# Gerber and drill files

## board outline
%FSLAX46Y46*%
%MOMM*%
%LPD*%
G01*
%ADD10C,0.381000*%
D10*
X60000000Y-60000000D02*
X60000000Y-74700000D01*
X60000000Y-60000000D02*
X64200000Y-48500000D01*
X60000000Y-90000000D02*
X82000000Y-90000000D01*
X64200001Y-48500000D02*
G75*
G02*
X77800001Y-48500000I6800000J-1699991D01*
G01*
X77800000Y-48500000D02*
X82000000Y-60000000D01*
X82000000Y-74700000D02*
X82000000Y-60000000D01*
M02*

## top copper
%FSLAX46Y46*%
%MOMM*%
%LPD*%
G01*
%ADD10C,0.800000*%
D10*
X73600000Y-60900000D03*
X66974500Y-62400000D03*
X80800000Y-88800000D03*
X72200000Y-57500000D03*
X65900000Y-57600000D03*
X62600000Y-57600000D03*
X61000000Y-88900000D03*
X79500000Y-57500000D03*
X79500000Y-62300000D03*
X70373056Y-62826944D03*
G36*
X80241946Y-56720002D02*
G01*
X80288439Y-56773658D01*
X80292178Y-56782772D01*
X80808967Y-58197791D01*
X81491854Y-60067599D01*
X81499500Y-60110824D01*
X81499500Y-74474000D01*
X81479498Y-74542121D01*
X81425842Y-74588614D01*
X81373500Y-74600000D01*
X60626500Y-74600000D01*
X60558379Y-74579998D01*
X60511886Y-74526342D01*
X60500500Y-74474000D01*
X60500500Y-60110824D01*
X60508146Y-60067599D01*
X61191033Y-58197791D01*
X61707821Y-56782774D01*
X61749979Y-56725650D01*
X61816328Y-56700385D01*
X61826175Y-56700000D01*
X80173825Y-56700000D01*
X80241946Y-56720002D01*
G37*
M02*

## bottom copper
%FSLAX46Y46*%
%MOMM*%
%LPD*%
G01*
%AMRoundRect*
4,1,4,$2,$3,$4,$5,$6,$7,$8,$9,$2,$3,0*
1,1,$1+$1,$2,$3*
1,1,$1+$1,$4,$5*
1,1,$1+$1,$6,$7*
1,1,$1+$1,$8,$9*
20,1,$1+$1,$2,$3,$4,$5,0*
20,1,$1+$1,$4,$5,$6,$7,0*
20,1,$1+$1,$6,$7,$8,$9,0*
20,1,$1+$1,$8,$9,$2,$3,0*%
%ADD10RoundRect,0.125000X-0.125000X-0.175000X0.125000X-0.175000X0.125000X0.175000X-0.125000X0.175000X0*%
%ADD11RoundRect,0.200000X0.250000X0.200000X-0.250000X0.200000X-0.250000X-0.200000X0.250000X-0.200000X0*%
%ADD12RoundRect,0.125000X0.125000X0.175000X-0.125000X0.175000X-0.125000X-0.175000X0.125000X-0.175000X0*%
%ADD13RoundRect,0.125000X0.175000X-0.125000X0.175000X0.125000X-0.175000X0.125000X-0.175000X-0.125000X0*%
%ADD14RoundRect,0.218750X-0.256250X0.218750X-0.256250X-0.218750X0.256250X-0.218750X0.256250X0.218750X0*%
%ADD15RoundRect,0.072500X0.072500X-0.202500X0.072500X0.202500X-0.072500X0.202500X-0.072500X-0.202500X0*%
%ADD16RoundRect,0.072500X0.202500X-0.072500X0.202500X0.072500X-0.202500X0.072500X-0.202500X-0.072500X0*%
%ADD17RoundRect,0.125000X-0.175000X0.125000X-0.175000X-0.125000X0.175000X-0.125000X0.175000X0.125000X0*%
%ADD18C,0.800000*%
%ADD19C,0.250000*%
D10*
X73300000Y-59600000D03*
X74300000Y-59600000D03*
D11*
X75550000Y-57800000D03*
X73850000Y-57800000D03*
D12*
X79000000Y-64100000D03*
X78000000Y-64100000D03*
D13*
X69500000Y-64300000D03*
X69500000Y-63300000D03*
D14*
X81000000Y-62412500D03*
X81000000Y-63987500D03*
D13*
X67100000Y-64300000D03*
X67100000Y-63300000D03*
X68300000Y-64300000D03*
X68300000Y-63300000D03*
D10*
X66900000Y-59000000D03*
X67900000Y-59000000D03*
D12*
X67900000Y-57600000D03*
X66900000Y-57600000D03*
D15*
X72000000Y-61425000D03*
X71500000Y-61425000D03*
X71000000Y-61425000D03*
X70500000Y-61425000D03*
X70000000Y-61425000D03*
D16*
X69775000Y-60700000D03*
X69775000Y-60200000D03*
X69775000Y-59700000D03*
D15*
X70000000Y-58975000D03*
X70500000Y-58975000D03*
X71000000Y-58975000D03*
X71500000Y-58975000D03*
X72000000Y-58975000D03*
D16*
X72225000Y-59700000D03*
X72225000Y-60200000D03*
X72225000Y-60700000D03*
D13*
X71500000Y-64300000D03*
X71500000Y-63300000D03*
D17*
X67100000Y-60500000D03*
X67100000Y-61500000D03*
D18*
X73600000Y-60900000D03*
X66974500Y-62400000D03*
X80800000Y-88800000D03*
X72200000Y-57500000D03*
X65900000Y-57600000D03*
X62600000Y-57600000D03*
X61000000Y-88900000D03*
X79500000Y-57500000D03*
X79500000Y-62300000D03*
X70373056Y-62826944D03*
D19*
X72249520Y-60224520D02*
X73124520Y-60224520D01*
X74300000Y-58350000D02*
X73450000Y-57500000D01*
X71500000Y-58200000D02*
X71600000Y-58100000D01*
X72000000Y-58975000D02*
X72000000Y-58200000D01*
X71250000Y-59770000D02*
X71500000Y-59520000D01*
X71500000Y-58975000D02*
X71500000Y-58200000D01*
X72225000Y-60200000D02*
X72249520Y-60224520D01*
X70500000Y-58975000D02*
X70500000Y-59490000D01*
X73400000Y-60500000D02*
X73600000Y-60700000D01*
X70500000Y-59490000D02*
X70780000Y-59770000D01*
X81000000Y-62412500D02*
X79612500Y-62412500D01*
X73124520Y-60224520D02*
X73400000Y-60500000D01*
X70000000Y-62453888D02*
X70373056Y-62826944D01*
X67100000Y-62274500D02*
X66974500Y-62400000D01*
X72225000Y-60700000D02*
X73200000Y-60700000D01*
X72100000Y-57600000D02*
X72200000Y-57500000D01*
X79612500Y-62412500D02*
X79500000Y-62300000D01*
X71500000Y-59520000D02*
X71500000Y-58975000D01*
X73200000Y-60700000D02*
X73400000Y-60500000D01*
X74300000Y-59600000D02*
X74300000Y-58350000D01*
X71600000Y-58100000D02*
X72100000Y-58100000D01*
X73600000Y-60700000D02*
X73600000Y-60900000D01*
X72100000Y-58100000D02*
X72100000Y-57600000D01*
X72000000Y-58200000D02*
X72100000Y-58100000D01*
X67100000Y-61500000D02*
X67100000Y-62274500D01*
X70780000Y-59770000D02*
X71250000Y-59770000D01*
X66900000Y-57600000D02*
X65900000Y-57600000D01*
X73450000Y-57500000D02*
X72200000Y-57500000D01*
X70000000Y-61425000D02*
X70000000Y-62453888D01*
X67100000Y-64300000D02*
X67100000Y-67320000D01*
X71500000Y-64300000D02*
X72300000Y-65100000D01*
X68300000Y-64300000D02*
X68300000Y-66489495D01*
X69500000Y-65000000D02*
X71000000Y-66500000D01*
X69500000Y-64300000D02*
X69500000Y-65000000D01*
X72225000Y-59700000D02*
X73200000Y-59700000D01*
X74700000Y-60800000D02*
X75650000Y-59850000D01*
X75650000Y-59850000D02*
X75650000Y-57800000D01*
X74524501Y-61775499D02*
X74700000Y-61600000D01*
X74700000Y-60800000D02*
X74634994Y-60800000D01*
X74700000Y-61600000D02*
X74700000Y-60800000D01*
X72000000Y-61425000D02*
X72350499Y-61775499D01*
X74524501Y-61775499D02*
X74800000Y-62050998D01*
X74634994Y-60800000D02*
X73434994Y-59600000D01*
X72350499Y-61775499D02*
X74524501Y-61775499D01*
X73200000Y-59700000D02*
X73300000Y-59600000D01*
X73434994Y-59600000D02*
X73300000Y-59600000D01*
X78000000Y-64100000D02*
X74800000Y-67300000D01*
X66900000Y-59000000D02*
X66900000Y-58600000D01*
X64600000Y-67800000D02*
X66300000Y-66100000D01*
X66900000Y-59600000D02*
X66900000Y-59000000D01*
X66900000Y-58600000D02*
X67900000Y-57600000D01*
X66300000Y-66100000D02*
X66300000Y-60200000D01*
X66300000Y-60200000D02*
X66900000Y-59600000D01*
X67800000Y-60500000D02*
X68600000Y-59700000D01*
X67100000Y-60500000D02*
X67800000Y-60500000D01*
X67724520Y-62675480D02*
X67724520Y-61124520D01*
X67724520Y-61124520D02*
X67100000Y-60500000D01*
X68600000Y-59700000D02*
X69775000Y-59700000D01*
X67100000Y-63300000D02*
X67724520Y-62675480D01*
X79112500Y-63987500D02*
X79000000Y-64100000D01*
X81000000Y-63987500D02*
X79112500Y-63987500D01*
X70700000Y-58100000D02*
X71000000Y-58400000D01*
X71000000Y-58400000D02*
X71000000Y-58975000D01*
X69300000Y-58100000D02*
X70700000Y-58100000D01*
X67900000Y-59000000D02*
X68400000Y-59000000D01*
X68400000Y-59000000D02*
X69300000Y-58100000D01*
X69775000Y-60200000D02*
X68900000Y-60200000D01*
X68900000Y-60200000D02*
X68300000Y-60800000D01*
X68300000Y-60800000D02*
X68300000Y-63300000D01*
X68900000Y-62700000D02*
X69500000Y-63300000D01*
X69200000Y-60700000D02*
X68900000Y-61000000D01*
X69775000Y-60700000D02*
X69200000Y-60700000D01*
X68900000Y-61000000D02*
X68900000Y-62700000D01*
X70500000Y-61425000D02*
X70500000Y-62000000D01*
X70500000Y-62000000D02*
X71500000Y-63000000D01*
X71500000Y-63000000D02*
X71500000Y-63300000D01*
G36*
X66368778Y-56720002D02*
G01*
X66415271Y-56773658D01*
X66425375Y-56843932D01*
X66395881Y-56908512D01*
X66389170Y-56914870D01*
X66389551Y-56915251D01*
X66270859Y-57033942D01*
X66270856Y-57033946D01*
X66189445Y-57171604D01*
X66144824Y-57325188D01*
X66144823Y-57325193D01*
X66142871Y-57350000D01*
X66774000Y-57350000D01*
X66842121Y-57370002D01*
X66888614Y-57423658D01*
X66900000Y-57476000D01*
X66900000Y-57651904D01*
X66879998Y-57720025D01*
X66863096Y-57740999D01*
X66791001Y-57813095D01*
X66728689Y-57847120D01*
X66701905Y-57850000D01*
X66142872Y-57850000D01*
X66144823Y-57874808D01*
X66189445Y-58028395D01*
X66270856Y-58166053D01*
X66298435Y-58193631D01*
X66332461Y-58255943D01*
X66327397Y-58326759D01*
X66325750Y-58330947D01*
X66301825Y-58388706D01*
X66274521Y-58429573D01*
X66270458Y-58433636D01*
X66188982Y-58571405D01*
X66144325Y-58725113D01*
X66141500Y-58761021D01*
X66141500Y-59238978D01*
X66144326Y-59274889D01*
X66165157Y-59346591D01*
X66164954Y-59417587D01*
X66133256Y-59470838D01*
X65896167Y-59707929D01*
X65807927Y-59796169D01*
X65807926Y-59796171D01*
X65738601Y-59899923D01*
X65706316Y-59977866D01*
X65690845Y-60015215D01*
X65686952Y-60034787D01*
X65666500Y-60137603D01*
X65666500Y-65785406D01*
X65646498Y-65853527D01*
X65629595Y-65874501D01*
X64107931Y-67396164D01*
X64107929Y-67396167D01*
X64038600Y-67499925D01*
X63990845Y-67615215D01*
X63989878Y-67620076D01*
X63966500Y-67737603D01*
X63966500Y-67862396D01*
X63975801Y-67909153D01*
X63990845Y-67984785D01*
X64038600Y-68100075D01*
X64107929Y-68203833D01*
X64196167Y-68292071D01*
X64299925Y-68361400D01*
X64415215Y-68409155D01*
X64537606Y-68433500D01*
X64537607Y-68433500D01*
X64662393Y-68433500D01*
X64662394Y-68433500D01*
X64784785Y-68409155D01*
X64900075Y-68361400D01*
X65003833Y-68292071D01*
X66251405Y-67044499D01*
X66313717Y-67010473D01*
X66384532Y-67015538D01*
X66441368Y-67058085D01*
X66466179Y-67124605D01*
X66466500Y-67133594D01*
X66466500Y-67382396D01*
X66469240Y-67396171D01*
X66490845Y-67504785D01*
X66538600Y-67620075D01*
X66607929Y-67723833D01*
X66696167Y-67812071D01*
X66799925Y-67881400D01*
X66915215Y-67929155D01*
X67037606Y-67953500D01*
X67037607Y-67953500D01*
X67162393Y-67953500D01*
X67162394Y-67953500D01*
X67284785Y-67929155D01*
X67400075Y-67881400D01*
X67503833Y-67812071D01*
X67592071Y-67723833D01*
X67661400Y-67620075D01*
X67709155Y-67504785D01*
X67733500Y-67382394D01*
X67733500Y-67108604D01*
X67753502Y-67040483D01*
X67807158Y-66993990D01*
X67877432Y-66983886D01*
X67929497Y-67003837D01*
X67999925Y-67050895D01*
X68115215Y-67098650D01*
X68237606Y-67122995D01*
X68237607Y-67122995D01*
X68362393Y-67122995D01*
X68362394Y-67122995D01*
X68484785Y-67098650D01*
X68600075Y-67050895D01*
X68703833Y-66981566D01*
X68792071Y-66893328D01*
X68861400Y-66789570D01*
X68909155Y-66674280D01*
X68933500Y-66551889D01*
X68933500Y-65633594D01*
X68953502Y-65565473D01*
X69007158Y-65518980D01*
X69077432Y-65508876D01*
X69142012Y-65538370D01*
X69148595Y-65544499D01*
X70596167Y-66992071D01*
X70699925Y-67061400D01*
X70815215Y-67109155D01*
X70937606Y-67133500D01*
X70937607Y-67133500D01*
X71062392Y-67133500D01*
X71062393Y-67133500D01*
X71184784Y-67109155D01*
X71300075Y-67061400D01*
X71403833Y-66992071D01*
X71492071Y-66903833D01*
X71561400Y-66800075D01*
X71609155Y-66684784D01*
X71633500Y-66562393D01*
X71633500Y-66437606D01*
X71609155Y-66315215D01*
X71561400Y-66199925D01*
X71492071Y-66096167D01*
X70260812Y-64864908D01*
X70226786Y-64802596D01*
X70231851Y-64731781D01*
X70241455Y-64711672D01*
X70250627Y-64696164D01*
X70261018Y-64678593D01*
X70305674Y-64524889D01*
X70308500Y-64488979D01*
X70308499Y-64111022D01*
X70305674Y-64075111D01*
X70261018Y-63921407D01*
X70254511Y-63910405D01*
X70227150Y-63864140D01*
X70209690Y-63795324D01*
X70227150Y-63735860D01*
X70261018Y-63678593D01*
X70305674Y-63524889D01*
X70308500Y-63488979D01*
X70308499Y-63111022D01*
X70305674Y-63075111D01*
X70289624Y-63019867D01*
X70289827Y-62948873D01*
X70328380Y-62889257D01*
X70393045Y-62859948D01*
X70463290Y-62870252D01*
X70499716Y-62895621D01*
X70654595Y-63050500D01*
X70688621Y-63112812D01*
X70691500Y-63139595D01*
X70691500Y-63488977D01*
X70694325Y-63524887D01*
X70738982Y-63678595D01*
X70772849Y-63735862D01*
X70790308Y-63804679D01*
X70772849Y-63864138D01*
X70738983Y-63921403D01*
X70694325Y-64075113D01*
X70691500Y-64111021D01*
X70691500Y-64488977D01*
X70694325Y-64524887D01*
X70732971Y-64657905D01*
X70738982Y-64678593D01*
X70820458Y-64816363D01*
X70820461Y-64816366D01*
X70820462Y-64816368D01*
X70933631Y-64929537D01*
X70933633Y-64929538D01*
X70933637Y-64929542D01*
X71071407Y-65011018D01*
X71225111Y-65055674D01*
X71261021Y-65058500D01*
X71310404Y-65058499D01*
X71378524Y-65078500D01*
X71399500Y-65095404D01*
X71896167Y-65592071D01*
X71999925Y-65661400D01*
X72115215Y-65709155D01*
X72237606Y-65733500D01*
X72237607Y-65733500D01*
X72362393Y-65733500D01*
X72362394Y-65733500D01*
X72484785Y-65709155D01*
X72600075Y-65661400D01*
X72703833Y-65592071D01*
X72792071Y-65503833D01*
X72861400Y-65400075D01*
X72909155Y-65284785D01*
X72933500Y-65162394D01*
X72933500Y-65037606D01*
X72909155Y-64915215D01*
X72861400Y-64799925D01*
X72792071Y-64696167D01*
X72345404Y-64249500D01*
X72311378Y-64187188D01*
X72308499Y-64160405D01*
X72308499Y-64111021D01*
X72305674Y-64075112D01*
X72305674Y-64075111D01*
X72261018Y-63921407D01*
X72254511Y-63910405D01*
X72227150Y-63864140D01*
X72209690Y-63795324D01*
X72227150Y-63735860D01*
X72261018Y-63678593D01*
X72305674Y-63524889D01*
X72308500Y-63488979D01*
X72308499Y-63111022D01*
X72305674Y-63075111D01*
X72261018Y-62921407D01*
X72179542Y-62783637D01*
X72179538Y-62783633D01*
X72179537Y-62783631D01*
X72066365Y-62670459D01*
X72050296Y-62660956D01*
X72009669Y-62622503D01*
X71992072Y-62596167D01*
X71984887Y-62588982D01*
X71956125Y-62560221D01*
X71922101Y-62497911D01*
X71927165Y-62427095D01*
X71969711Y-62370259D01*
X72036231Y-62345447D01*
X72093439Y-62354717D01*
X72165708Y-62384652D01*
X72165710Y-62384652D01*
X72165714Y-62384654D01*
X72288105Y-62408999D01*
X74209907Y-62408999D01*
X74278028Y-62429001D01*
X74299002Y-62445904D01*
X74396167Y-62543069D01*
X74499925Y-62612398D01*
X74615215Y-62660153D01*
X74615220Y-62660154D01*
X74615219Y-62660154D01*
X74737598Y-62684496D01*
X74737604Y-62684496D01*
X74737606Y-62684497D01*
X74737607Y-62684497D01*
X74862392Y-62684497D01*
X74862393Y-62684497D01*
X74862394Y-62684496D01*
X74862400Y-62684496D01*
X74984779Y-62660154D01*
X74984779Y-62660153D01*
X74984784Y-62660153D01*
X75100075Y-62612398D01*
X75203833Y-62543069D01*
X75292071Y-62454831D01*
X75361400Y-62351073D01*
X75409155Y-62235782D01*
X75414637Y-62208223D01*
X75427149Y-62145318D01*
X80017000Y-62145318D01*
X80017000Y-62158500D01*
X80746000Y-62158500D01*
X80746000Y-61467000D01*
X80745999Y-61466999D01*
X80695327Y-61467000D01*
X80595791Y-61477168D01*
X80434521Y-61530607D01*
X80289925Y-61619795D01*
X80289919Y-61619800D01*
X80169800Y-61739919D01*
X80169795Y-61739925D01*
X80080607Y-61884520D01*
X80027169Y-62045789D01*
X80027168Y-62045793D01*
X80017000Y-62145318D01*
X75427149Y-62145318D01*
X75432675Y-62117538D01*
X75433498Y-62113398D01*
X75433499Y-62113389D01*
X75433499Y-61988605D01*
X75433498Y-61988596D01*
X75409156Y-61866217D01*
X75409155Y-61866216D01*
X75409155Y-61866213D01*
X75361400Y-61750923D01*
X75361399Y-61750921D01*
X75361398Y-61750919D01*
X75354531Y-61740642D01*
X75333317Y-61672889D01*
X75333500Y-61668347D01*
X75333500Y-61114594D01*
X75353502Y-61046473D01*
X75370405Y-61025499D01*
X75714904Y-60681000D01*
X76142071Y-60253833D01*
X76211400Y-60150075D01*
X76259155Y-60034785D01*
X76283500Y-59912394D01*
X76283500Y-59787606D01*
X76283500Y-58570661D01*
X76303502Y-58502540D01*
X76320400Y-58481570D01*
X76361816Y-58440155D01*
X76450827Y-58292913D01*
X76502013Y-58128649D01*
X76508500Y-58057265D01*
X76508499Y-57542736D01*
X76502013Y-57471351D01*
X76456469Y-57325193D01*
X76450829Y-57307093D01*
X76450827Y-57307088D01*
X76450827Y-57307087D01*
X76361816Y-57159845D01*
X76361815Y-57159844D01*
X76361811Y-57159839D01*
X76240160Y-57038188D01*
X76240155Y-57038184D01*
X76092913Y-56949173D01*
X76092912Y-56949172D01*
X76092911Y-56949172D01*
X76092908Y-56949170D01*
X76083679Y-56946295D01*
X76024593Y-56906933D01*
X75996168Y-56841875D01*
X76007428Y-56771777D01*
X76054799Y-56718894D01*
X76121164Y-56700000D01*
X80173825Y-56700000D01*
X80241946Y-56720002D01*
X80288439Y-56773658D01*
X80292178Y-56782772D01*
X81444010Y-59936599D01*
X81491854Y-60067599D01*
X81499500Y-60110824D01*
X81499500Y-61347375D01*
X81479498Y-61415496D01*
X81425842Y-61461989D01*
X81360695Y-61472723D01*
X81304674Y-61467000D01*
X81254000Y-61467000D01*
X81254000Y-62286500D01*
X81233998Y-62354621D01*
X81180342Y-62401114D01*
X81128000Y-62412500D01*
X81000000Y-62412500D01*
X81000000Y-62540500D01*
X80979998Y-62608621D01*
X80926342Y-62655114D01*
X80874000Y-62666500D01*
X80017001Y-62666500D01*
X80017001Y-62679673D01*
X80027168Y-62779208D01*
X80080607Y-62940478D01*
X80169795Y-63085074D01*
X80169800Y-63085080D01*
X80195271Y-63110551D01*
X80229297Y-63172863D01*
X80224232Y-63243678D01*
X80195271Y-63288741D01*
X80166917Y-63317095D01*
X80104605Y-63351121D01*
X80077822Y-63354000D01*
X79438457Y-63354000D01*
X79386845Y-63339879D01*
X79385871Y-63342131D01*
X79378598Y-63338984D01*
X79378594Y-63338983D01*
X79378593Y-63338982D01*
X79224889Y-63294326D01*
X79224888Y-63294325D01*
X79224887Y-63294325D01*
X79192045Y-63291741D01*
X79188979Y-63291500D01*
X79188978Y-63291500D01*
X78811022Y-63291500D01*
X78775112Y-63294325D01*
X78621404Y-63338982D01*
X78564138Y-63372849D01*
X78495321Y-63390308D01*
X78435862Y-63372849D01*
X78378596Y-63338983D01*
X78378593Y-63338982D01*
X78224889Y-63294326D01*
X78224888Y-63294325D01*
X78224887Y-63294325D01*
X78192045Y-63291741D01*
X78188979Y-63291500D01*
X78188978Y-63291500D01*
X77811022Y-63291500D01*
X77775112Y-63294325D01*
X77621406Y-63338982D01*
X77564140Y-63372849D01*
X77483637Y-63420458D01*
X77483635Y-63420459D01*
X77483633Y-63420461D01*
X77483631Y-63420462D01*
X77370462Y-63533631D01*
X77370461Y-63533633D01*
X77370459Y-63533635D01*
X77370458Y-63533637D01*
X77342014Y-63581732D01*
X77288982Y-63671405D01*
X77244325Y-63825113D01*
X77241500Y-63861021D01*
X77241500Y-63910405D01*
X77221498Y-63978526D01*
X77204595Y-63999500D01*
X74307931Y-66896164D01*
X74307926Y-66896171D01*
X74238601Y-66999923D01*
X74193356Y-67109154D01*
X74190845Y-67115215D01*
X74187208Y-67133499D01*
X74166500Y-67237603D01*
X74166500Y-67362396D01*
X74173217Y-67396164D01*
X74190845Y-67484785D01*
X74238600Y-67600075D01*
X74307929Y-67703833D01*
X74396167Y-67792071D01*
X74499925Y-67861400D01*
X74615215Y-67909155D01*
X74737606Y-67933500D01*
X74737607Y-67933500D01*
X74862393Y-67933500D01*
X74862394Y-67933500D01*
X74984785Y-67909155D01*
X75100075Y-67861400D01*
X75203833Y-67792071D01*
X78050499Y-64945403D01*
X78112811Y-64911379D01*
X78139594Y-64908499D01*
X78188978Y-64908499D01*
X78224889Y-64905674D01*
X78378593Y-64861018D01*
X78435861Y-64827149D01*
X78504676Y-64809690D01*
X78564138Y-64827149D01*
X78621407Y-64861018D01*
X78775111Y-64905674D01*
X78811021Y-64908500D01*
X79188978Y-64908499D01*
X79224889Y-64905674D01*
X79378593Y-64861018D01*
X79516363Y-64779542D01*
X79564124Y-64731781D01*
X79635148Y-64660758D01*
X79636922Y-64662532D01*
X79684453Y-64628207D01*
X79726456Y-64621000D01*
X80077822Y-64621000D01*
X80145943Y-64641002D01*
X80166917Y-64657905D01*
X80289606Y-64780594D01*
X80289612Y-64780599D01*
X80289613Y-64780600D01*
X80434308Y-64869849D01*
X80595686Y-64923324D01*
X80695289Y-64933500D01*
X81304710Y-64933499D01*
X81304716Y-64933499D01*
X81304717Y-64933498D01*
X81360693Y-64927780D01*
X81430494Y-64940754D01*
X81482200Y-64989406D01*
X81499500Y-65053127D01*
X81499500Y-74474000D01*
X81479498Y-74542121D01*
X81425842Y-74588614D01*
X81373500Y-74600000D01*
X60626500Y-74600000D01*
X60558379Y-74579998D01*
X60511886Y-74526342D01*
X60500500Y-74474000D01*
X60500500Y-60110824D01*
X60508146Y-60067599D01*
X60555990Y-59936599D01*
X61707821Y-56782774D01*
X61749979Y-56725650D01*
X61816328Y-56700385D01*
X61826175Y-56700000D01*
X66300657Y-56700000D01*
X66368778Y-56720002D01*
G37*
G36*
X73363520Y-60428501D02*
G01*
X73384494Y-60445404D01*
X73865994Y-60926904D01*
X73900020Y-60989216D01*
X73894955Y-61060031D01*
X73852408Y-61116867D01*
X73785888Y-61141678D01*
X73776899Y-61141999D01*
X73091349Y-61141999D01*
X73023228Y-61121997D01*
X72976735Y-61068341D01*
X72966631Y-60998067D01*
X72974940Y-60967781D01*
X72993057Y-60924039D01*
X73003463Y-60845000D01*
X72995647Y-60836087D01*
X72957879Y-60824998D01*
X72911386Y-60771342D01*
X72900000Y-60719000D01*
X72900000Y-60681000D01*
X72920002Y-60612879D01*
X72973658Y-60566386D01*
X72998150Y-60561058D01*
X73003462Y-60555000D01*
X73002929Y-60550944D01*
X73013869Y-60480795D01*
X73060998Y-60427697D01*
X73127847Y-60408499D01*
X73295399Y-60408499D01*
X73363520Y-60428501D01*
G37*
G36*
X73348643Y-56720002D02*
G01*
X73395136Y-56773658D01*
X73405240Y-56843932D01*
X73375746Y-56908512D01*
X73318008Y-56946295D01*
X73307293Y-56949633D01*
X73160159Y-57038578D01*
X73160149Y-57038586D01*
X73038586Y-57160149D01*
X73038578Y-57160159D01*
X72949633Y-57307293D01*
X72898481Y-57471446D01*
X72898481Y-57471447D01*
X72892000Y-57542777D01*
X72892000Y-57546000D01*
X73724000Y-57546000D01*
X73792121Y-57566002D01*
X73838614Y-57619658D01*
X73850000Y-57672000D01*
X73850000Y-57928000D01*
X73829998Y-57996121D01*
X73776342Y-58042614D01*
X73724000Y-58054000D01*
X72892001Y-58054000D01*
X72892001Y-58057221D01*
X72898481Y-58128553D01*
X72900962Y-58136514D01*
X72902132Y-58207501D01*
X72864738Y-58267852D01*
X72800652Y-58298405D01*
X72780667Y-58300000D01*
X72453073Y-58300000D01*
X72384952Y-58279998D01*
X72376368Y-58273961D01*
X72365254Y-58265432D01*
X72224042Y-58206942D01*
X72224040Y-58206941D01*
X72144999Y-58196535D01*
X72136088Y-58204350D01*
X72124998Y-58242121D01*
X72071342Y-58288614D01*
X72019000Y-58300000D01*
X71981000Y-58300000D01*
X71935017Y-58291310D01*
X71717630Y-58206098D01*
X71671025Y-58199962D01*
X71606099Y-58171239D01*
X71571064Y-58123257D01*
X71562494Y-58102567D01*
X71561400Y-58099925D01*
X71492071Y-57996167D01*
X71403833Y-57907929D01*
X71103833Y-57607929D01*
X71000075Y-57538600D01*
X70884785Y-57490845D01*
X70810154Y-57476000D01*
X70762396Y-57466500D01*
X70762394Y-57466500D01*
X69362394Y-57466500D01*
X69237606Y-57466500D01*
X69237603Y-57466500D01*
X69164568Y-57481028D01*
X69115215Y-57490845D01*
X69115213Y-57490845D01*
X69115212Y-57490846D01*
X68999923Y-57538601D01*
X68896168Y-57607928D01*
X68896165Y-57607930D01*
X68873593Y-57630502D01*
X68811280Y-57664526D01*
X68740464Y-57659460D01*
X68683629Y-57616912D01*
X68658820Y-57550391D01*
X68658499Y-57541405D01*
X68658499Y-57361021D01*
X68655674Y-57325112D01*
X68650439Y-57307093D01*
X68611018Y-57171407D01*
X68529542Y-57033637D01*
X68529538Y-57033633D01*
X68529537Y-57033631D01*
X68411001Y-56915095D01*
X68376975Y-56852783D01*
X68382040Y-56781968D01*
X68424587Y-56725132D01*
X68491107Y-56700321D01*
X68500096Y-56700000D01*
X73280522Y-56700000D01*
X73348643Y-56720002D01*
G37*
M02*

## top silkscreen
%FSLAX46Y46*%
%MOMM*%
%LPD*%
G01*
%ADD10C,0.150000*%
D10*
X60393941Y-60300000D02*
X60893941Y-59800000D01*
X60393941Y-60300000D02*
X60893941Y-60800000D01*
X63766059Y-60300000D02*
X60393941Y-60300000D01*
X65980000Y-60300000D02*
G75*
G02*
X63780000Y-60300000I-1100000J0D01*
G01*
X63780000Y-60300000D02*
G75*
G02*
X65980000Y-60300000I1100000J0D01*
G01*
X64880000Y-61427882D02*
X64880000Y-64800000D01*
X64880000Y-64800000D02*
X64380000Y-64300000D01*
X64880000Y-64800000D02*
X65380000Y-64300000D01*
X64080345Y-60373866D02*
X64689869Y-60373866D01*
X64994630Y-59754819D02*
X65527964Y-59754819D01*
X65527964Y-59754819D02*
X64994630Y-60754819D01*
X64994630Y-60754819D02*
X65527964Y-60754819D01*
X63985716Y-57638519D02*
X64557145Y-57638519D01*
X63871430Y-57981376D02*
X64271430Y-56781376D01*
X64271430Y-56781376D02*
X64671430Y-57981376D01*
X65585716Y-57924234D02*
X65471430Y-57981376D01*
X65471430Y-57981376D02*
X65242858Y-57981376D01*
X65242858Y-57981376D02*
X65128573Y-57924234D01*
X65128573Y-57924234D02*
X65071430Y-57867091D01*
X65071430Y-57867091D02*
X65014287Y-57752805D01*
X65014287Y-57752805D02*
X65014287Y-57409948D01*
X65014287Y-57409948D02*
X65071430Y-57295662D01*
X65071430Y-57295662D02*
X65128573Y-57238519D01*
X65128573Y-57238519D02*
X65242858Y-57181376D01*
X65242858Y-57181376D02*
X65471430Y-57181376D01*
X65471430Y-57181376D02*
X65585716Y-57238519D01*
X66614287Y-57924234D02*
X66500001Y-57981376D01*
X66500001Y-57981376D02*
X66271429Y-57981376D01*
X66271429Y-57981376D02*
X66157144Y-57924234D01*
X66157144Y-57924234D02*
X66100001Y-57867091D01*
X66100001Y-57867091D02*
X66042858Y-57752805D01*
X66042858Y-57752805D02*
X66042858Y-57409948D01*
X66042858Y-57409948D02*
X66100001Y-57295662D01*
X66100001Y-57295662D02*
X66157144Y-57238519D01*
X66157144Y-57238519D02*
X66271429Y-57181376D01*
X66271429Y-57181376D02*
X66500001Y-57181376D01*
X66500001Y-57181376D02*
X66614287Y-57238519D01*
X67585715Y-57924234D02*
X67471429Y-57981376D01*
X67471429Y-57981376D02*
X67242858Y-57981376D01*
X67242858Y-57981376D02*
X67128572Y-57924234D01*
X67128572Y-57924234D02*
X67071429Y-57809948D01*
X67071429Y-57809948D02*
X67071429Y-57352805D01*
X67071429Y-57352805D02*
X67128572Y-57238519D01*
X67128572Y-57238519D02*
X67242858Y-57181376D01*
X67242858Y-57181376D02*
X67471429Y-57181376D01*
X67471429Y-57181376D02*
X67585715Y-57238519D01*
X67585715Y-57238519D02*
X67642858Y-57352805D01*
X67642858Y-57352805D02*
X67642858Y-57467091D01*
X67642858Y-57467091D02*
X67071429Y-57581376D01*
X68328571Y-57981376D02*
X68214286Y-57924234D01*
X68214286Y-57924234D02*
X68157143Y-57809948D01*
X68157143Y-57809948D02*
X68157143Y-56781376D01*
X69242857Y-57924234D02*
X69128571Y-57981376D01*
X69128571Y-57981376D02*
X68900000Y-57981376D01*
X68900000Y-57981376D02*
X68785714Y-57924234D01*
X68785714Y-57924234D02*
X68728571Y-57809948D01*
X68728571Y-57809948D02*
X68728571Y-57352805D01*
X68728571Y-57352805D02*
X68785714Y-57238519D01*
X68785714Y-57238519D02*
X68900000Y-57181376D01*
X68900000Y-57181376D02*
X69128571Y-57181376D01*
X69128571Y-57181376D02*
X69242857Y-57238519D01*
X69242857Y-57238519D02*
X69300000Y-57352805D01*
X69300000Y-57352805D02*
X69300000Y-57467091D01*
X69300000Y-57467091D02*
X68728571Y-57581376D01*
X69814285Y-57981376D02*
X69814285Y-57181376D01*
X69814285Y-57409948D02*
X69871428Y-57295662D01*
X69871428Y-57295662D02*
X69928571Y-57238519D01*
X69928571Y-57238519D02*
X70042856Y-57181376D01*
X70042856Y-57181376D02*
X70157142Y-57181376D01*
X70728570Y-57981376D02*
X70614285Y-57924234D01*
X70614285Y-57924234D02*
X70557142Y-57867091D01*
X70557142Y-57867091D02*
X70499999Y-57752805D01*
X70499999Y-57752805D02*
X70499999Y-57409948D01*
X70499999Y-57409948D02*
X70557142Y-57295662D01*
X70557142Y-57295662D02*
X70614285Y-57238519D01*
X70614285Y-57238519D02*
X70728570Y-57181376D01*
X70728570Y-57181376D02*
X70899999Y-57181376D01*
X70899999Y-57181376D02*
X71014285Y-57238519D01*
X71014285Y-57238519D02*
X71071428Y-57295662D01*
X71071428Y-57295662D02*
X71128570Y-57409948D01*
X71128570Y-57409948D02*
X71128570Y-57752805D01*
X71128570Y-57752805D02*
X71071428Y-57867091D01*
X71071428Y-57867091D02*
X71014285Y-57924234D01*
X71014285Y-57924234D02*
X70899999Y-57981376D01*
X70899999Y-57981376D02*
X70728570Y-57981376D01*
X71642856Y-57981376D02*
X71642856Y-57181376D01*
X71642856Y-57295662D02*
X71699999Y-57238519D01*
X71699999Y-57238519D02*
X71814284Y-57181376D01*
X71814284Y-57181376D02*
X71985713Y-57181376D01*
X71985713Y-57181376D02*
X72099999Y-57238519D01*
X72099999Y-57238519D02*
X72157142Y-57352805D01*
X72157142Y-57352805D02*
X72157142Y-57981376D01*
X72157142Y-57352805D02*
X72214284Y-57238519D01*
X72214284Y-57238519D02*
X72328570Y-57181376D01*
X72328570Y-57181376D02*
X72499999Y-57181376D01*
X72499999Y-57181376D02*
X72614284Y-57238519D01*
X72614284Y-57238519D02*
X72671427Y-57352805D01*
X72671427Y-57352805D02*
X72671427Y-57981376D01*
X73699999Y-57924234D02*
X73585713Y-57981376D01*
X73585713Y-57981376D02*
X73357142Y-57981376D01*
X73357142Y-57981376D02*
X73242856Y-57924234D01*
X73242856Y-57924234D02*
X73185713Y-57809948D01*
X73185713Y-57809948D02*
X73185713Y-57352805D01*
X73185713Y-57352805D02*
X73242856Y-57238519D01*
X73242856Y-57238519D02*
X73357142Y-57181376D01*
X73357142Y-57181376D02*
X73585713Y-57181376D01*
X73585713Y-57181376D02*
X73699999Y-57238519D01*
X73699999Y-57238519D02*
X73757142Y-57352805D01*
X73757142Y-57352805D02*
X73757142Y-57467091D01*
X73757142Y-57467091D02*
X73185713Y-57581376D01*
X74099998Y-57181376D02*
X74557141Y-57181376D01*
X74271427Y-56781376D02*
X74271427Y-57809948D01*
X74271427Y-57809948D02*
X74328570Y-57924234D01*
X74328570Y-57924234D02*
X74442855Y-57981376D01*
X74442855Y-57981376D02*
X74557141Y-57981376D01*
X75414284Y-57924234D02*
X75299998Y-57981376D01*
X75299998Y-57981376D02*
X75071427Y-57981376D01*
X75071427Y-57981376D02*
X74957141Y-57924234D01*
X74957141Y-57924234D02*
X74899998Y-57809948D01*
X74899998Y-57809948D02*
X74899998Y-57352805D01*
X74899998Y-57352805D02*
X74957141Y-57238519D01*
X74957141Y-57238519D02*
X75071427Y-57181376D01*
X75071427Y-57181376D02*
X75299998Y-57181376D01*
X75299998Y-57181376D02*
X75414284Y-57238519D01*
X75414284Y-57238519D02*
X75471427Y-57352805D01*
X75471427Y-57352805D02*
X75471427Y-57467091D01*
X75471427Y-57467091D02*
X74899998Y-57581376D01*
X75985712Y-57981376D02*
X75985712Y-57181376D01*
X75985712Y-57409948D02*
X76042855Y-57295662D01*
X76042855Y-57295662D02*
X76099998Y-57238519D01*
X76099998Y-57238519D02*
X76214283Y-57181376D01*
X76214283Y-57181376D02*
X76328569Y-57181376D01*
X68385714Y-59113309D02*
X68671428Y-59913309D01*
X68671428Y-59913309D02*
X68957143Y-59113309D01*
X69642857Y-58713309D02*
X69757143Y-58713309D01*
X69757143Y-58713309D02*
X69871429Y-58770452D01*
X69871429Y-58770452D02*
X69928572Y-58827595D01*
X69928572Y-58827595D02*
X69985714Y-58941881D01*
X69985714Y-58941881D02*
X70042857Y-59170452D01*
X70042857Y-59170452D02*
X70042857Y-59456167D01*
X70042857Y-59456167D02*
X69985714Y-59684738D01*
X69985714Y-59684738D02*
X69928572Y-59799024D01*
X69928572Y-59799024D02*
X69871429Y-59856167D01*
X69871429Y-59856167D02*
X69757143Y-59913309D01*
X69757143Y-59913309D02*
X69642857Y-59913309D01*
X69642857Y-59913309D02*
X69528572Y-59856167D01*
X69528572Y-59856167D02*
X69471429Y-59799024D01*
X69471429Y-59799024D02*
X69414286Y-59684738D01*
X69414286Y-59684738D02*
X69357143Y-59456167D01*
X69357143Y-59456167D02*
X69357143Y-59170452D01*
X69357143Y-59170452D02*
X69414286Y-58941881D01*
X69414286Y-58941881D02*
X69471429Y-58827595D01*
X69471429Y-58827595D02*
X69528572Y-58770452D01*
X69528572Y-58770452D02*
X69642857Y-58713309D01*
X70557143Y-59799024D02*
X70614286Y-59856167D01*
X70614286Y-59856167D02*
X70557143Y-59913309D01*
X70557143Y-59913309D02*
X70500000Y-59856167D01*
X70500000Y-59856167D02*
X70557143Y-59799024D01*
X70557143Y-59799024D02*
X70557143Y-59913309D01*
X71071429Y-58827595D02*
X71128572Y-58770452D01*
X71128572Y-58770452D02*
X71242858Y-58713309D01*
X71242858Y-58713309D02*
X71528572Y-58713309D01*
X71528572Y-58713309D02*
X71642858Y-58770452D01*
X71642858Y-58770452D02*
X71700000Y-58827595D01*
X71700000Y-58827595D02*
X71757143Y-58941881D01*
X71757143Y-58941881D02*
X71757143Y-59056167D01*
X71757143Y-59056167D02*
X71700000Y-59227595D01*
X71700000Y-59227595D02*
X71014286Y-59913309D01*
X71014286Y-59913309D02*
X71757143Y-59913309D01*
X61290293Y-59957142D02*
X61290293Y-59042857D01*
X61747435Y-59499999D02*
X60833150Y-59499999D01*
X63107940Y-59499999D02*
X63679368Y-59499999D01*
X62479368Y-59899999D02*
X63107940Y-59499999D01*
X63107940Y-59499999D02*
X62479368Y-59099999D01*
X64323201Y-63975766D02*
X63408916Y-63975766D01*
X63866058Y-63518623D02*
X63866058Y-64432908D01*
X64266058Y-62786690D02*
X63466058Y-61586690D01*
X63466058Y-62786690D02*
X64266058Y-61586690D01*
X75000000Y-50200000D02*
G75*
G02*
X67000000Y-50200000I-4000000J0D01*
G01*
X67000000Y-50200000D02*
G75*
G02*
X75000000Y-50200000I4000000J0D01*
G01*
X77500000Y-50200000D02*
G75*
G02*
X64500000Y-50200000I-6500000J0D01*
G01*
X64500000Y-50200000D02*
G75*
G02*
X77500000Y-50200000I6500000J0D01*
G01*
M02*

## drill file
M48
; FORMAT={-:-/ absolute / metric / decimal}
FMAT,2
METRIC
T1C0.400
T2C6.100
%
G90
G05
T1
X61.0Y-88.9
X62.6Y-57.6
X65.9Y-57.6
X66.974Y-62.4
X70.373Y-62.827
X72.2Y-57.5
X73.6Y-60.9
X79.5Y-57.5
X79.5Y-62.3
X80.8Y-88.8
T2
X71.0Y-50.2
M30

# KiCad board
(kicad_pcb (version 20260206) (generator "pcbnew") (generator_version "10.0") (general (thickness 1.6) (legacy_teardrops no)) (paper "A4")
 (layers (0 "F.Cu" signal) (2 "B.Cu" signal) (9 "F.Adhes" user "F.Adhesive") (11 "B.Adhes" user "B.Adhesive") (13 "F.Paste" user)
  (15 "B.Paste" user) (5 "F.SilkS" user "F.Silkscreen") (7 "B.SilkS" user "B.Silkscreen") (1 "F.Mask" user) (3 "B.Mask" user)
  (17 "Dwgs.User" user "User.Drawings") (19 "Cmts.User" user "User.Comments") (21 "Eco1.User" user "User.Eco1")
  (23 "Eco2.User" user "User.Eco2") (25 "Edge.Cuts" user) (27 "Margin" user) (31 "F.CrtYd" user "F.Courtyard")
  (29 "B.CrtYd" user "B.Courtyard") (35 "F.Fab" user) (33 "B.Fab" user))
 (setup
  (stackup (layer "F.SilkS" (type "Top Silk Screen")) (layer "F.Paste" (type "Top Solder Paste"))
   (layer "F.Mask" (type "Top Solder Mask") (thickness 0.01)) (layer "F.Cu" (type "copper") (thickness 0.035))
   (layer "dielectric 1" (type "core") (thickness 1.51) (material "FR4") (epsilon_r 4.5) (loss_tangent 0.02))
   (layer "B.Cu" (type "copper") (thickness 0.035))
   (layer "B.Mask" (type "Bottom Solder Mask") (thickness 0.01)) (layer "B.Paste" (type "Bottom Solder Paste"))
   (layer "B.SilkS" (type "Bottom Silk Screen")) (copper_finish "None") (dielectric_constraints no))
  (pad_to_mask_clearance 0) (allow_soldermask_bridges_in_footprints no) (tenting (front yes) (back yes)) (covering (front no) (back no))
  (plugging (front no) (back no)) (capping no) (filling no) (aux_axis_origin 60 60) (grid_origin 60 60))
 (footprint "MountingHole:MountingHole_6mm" (layer "F.Cu") (at 71 50.2)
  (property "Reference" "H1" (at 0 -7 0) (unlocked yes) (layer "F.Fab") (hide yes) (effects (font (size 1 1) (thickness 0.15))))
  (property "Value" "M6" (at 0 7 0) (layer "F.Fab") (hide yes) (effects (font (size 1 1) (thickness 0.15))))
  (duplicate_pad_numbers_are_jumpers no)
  (fp_circle (center 0 0) (end 4 0) (stroke (width 0.15) (type solid)) (fill no) (layer "F.SilkS"))
  (fp_circle (center 0 0) (end 6.5 0) (stroke (width 0.15) (type solid)) (fill no) (layer "F.SilkS"))
  (pad "" np_thru_hole circle (at 0 0) (size 6.1 6.1) (drill 6.1) (layers "*.Cu" "*.Mask")))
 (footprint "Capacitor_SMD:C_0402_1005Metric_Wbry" (layer "B.Cu") (at 73.8 59.6)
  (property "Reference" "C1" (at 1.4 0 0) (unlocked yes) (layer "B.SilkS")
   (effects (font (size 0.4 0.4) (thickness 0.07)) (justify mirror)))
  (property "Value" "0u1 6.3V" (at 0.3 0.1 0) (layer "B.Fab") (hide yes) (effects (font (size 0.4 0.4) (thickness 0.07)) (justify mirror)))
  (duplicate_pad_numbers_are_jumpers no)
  (pad "1" smd roundrect (at -0.5 0) (size 0.5 0.6) (layers "B.Cu" "B.Mask" "B.Paste") (roundrect_rratio 0.25) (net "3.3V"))
  (pad "2" smd roundrect (at 0.5 0) (size 0.5 0.6) (layers "B.Cu" "B.Mask" "B.Paste") (roundrect_rratio 0.25) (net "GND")))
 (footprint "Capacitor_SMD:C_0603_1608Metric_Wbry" (layer "B.Cu") (at 74.7 57.8 180)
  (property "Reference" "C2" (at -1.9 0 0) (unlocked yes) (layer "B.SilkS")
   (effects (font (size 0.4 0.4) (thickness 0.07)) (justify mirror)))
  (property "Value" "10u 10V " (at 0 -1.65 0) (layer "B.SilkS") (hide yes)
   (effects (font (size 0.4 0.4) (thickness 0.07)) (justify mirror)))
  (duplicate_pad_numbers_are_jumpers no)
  (pad "1" smd roundrect (at -0.85 0 180) (size 0.9 0.8) (layers "B.Cu" "B.Mask" "B.Paste") (roundrect_rratio 0.25) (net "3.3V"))
  (pad "2" smd roundrect (at 0.85 0 180) (size 0.9 0.8) (layers "B.Cu" "B.Mask" "B.Paste") (roundrect_rratio 0.25) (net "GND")))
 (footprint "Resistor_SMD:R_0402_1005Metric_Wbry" (layer "B.Cu") (at 78.5 64.1 180)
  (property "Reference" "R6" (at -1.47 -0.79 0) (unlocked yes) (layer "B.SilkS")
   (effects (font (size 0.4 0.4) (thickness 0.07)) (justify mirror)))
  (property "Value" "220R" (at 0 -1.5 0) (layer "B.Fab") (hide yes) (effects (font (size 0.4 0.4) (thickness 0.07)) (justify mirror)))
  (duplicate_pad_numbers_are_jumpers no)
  (pad "1" smd roundrect (at -0.5 0 180) (size 0.5 0.6) (layers "B.Cu" "B.Mask" "B.Paste") (roundrect_rratio 0.25) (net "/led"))
  (pad "2" smd roundrect (at 0.5 0 180) (size 0.5 0.6) (layers "B.Cu" "B.Mask" "B.Paste") (roundrect_rratio 0.25) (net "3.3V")))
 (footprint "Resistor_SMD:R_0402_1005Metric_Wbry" (layer "B.Cu") (at 69.5 63.8 90)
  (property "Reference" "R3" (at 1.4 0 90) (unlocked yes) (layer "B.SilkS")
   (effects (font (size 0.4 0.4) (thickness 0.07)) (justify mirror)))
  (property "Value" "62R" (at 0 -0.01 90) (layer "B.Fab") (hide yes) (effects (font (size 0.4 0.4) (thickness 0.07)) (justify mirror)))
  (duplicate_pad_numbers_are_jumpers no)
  (pad "1" smd roundrect (at -0.5 0 90) (size 0.5 0.6) (layers "B.Cu" "B.Mask" "B.Paste") (roundrect_rratio 0.25) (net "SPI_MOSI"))
  (pad "2" smd roundrect (at 0.5 0 90) (size 0.5 0.6) (layers "B.Cu" "B.Mask" "B.Paste") (roundrect_rratio 0.25) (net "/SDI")))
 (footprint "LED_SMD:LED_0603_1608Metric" (layer "B.Cu") (at 81 63.2 -90)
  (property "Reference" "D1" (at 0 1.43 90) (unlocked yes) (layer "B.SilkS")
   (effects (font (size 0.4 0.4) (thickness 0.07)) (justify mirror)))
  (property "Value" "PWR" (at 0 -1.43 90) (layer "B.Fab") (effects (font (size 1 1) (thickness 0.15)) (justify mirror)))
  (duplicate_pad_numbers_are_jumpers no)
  (pad "1" smd roundrect (at -0.7875 0 270) (size 0.875 0.95) (layers "B.Cu" "B.Mask" "B.Paste") (roundrect_rratio 0.25) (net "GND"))
  (pad "2" smd roundrect (at 0.7875 0 270) (size 0.875 0.95) (layers "B.Cu" "B.Mask" "B.Paste") (roundrect_rratio 0.25) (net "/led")))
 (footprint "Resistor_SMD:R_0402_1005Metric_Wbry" (layer "B.Cu") (at 67.1 63.8 90)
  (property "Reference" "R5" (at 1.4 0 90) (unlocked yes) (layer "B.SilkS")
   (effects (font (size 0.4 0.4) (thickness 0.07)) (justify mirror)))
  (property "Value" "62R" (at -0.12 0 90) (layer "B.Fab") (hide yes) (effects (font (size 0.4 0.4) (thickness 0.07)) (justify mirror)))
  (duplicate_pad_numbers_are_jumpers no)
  (pad "1" smd roundrect (at -0.5 0 90) (size 0.5 0.6) (layers "B.Cu" "B.Mask" "B.Paste") (roundrect_rratio 0.25) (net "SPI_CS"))
  (pad "2" smd roundrect (at 0.5 0 90) (size 0.5 0.6) (layers "B.Cu" "B.Mask" "B.Paste") (roundrect_rratio 0.25) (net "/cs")))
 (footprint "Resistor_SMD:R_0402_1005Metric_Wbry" (layer "B.Cu") (at 68.3 63.8 90)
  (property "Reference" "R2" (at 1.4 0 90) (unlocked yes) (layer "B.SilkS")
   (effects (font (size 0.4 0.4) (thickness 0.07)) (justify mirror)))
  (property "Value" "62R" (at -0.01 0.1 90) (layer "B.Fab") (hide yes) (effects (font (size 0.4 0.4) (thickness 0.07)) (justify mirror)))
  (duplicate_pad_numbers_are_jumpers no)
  (pad "1" smd roundrect (at -0.5 0 90) (size 0.5 0.6) (layers "B.Cu" "B.Mask" "B.Paste") (roundrect_rratio 0.25) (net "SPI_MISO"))
  (pad "2" smd roundrect (at 0.5 0 90) (size 0.5 0.6) (layers "B.Cu" "B.Mask" "B.Paste") (roundrect_rratio 0.25) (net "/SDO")))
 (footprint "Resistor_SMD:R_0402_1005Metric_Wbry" (layer "B.Cu") (at 67.4 59)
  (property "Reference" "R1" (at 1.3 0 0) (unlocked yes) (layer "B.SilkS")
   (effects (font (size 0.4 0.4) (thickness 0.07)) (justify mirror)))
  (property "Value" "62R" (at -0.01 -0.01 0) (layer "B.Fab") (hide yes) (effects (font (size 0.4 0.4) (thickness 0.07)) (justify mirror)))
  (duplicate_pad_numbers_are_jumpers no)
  (pad "1" smd roundrect (at -0.5 0) (size 0.5 0.6) (layers "B.Cu" "B.Mask" "B.Paste") (roundrect_rratio 0.25) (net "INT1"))
  (pad "2" smd roundrect (at 0.5 0) (size 0.5 0.6) (layers "B.Cu" "B.Mask" "B.Paste") (roundrect_rratio 0.25) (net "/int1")))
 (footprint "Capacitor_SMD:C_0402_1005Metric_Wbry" (layer "B.Cu") (at 67.4 57.6 180)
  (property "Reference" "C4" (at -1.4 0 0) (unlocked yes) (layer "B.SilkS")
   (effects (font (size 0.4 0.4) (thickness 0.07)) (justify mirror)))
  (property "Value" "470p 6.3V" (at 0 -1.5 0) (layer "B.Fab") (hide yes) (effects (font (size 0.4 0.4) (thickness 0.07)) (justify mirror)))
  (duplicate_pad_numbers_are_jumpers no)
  (pad "1" smd roundrect (at -0.5 0 180) (size 0.5 0.6) (layers "B.Cu" "B.Mask" "B.Paste") (roundrect_rratio 0.25) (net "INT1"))
  (pad "2" smd roundrect (at 0.5 0 180) (size 0.5 0.6) (layers "B.Cu" "B.Mask" "B.Paste") (roundrect_rratio 0.25) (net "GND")))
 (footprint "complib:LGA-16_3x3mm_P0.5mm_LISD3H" (layer "B.Cu") (at 71 60.2 90)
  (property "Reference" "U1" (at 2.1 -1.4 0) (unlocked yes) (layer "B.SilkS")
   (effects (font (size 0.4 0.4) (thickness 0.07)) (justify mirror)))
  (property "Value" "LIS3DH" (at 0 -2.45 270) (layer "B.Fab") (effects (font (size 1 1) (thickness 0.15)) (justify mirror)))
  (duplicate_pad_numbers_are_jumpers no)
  (pad "1" smd roundrect (at -1.225 1 90) (size 0.55 0.29) (layers "B.Cu" "B.Mask" "B.Paste") (roundrect_rratio 0.25) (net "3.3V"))
  (pad "2" smd roundrect (at -1.225 0.5 90) (size 0.55 0.29) (layers "B.Cu" "B.Mask" "B.Paste") (roundrect_rratio 0.25)
   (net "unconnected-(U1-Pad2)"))
  (pad "3" smd roundrect (at -1.225 0 90) (size 0.55 0.29) (layers "B.Cu" "B.Mask" "B.Paste") (roundrect_rratio 0.25)
   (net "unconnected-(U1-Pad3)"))
  (pad "4" smd roundrect (at -1.225 -0.5 90) (size 0.55 0.29) (layers "B.Cu" "B.Mask" "B.Paste") (roundrect_rratio 0.25) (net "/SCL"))
  (pad "5" smd roundrect (at -1.225 -1 90) (size 0.55 0.29) (layers "B.Cu" "B.Mask" "B.Paste") (roundrect_rratio 0.25) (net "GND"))
  (pad "6" smd roundrect (at -0.5 -1.225 90) (size 0.29 0.55) (layers "B.Cu" "B.Mask" "B.Paste") (roundrect_rratio 0.25) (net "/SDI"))
  (pad "7" smd roundrect (at 0 -1.225 90) (size 0.29 0.55) (layers "B.Cu" "B.Mask" "B.Paste") (roundrect_rratio 0.25) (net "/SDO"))
  (pad "8" smd roundrect (at 0.5 -1.225 90) (size 0.29 0.55) (layers "B.Cu" "B.Mask" "B.Paste") (roundrect_rratio 0.25) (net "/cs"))
  (pad "9" smd roundrect (at 1.225 -1 90) (size 0.55 0.29) (layers "B.Cu" "B.Mask" "B.Paste") (roundrect_rratio 0.25)
   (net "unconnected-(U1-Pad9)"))
  (pad "10" smd roundrect (at 1.225 -0.5 90) (size 0.55 0.29) (layers "B.Cu" "B.Mask" "B.Paste") (roundrect_rratio 0.25) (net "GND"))
  (pad "11" smd roundrect (at 1.225 0 90) (size 0.55 0.29) (layers "B.Cu" "B.Mask" "B.Paste") (roundrect_rratio 0.25) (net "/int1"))
  (pad "12" smd roundrect (at 1.225 0.5 90) (size 0.55 0.29) (layers "B.Cu" "B.Mask" "B.Paste") (roundrect_rratio 0.25) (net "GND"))
  (pad "13" smd roundrect (at 1.225 1 90) (size 0.55 0.29) (layers "B.Cu" "B.Mask" "B.Paste") (roundrect_rratio 0.25) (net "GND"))
  (pad "14" smd roundrect (at 0.5 1.225 90) (size 0.29 0.55) (layers "B.Cu" "B.Mask" "B.Paste") (roundrect_rratio 0.25) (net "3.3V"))
  (pad "15" smd roundrect (at 0 1.225 90) (size 0.29 0.55) (layers "B.Cu" "B.Mask" "B.Paste") (roundrect_rratio 0.25) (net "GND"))
  (pad "16" smd roundrect (at -0.5 1.225 90) (size 0.29 0.55) (layers "B.Cu" "B.Mask" "B.Paste") (roundrect_rratio 0.25) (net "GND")))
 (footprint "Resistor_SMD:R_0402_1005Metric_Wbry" (layer "B.Cu") (at 71.5 63.8 90)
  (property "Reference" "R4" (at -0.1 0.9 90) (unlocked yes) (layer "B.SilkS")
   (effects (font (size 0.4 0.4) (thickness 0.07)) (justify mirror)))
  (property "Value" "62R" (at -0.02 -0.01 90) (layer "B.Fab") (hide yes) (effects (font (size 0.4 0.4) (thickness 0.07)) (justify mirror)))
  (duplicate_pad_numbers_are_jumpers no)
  (pad "1" smd roundrect (at -0.5 0 90) (size 0.5 0.6) (layers "B.Cu" "B.Mask" "B.Paste") (roundrect_rratio 0.25) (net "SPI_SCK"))
  (pad "2" smd roundrect (at 0.5 0 90) (size 0.5 0.6) (layers "B.Cu" "B.Mask" "B.Paste") (roundrect_rratio 0.25) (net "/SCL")))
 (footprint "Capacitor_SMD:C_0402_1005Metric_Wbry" (layer "B.Cu") (at 67.1 61 -90)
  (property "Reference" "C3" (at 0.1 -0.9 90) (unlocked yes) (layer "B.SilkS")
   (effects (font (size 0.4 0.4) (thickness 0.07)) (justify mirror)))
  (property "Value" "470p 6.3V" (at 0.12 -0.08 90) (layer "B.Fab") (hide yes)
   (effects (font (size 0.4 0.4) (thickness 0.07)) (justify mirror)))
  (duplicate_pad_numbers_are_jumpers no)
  (pad "1" smd roundrect (at -0.5 0 270) (size 0.5 0.6) (layers "B.Cu" "B.Mask" "B.Paste") (roundrect_rratio 0.25) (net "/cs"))
  (pad "2" smd roundrect (at 0.5 0 270) (size 0.5 0.6) (layers "B.Cu" "B.Mask" "B.Paste") (roundrect_rratio 0.25) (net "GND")))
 (gr_line (start 60.393941 60.3) (end 60.893941 59.8) (stroke (width 0.15) (type solid)) (layer "F.SilkS"))
 (gr_line (start 60.393941 60.3) (end 60.893941 60.8) (stroke (width 0.15) (type solid)) (layer "F.SilkS"))
 (gr_line (start 63.766059 60.3) (end 60.393941 60.3) (stroke (width 0.15) (type solid)) (layer "F.SilkS"))
 (gr_circle (center 64.88 60.3) (end 65.98 60.3) (stroke (width 0.15) (type solid)) (fill no) (layer "F.SilkS"))
 (gr_line (start 64.88 61.427882) (end 64.88 64.8) (stroke (width 0.15) (type solid)) (layer "F.SilkS"))
 (gr_line (start 64.88 64.8) (end 64.38 64.3) (stroke (width 0.15) (type solid)) (layer "F.SilkS"))
 (gr_line (start 64.88 64.8) (end 65.38 64.3) (stroke (width 0.15) (type solid)) (layer "F.SilkS"))
 (gr_line (start 60 60) (end 60 74.7) (stroke (width 0.381) (type solid)) (layer "Edge.Cuts"))
 (gr_line (start 60 60) (end 64.2 48.5) (stroke (width 0.381) (type solid)) (layer "Edge.Cuts"))
 (gr_line (start 60 90) (end 82 90) (stroke (width 0.381) (type solid)) (layer "Edge.Cuts"))
 (gr_arc (start 64.200001 48.5) (mid 71.000001 43.190714) (end 77.8 48.5) (stroke (width 0.381) (type solid)) (layer "Edge.Cuts"))
 (gr_line (start 77.8 48.5) (end 82 60) (stroke (width 0.381) (type solid)) (layer "Edge.Cuts"))
 (gr_line (start 82 74.7) (end 82 60) (stroke (width 0.381) (type solid)) (layer "Edge.Cuts"))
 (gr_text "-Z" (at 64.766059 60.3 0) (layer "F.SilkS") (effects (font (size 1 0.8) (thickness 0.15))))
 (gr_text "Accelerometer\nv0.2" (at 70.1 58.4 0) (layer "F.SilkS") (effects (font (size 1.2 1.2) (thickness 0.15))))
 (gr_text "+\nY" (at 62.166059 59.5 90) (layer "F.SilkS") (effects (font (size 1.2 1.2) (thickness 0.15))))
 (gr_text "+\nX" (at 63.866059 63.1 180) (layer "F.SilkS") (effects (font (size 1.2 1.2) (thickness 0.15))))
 (via (at 73.6 60.9) (size 0.8) (drill 0.4) (layers "F.Cu" "B.Cu") (capping no) (covering (front no) (back no))
  (plugging (front no) (back no)) (filling no) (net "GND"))
 (via (at 66.9745 62.4) (size 0.8) (drill 0.4) (layers "F.Cu" "B.Cu") (capping no) (covering (front no) (back no))
  (plugging (front no) (back no)) (filling no) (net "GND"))
 (via (at 80.8 88.8) (size 0.8) (drill 0.4) (layers "F.Cu" "B.Cu") (free yes) (capping no) (covering (front no) (back no))
  (plugging (front no) (back no)) (filling no) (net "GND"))
 (via (at 72.2 57.5) (size 0.8) (drill 0.4) (layers "F.Cu" "B.Cu") (capping no) (covering (front no) (back no))
  (plugging (front no) (back no)) (filling no) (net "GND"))
 (via (at 65.9 57.6) (size 0.8) (drill 0.4) (layers "F.Cu" "B.Cu") (capping no) (covering (front no) (back no))
  (plugging (front no) (back no)) (filling no) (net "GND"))
 (via (at 62.6 57.6) (size 0.8) (drill 0.4) (layers "F.Cu" "B.Cu") (free yes) (capping no) (covering (front no) (back no))
  (plugging (front no) (back no)) (filling no) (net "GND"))
 (via (at 61 88.9) (size 0.8) (drill 0.4) (layers "F.Cu" "B.Cu") (free yes) (capping no) (covering (front no) (back no))
  (plugging (front no) (back no)) (filling no) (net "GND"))
 (via (at 79.5 57.5) (size 0.8) (drill 0.4) (layers "F.Cu" "B.Cu") (free yes) (capping no) (covering (front no) (back no))
  (plugging (front no) (back no)) (filling no) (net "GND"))
 (via (at 79.5 62.3) (size 0.8) (drill 0.4) (layers "F.Cu" "B.Cu") (capping no) (covering (front no) (back no))
  (plugging (front no) (back no)) (filling no) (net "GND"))
 (via (at 70.373056 62.826944) (size 0.8) (drill 0.4) (layers "F.Cu" "B.Cu") (capping no) (covering (front no) (back no))
  (plugging (front no) (back no)) (filling no) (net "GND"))
 (segment (start 72.24952 60.22452) (end 73.12452 60.22452) (width 0.25) (layer "B.Cu") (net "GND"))
 (segment (start 74.3 58.35) (end 73.45 57.5) (width 0.25) (layer "B.Cu") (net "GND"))
 (segment (start 71.5 58.2) (end 71.6 58.1) (width 0.25) (layer "B.Cu") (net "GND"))
 (segment (start 72 58.975) (end 72 58.2) (width 0.25) (layer "B.Cu") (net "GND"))
 (segment (start 71.25 59.77) (end 71.5 59.52) (width 0.25) (layer "B.Cu") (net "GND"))
 (segment (start 71.5 58.975) (end 71.5 58.2) (width 0.25) (layer "B.Cu") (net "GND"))
 (segment (start 72.225 60.2) (end 72.24952 60.22452) (width 0.25) (layer "B.Cu") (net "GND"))
 (segment (start 70.5 58.975) (end 70.5 59.49) (width 0.25) (layer "B.Cu") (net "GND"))
 (segment (start 73.4 60.5) (end 73.6 60.7) (width 0.25) (layer "B.Cu") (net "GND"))
 (segment (start 70.5 59.49) (end 70.78 59.77) (width 0.25) (layer "B.Cu") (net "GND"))
 (segment (start 81 62.4125) (end 79.6125 62.4125) (width 0.25) (layer "B.Cu") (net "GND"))
 (segment (start 73.12452 60.22452) (end 73.4 60.5) (width 0.25) (layer "B.Cu") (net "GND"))
 (segment (start 70 62.453888) (end 70.373056 62.826944) (width 0.25) (layer "B.Cu") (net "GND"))
 (segment (start 67.1 62.2745) (end 66.9745 62.4) (width 0.25) (layer "B.Cu") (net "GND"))
 (segment (start 72.225 60.7) (end 73.2 60.7) (width 0.25) (layer "B.Cu") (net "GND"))
 (segment (start 72.1 57.6) (end 72.2 57.5) (width 0.25) (layer "B.Cu") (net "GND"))
 (segment (start 79.6125 62.4125) (end 79.5 62.3) (width 0.25) (layer "B.Cu") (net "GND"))
 (segment (start 71.5 59.52) (end 71.5 58.975) (width 0.25) (layer "B.Cu") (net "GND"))
 (segment (start 73.2 60.7) (end 73.4 60.5) (width 0.25) (layer "B.Cu") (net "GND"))
 (segment (start 74.3 59.6) (end 74.3 58.35) (width 0.25) (layer "B.Cu") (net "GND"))
 (segment (start 71.6 58.1) (end 72.1 58.1) (width 0.25) (layer "B.Cu") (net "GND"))
 (segment (start 73.6 60.7) (end 73.6 60.9) (width 0.25) (layer "B.Cu") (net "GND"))
 (segment (start 72.1 58.1) (end 72.1 57.6) (width 0.25) (layer "B.Cu") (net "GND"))
 (segment (start 72 58.2) (end 72.1 58.1) (width 0.25) (layer "B.Cu") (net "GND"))
 (segment (start 67.1 61.5) (end 67.1 62.2745) (width 0.25) (layer "B.Cu") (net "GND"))
 (segment (start 70.78 59.77) (end 71.25 59.77) (width 0.25) (layer "B.Cu") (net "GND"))
 (segment (start 66.9 57.6) (end 65.9 57.6) (width 0.25) (layer "B.Cu") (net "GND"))
 (segment (start 73.45 57.5) (end 72.2 57.5) (width 0.25) (layer "B.Cu") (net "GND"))
 (segment (start 70 61.425) (end 70 62.453888) (width 0.25) (layer "B.Cu") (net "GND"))
 (segment (start 67.1 64.3) (end 67.1 67.32) (width 0.25) (layer "B.Cu") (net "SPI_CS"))
 (segment (start 71.5 64.3) (end 72.3 65.1) (width 0.25) (layer "B.Cu") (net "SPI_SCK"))
 (segment (start 68.3 64.3) (end 68.3 66.489495) (width 0.25) (layer "B.Cu") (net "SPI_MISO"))
 (segment (start 69.5 65) (end 71 66.5) (width 0.25) (layer "B.Cu") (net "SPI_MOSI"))
 (segment (start 69.5 64.3) (end 69.5 65) (width 0.25) (layer "B.Cu") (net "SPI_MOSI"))
 (segment (start 72.225 59.7) (end 73.2 59.7) (width 0.25) (layer "B.Cu") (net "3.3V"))
 (segment (start 74.7 60.8) (end 75.65 59.85) (width 0.25) (layer "B.Cu") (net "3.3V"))
 (segment (start 75.65 59.85) (end 75.65 57.8) (width 0.25) (layer "B.Cu") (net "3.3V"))
 (segment (start 74.524501 61.775499) (end 74.7 61.6) (width 0.25) (layer "B.Cu") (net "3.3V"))
 (segment (start 74.7 60.8) (end 74.634994 60.8) (width 0.25) (layer "B.Cu") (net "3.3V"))
 (segment (start 74.7 61.6) (end 74.7 60.8) (width 0.25) (layer "B.Cu") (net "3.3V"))
 (segment (start 72 61.425) (end 72.350499 61.775499) (width 0.25) (layer "B.Cu") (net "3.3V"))
 (segment (start 74.524501 61.775499) (end 74.8 62.050998) (width 0.25) (layer "B.Cu") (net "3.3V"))
 (segment (start 74.634994 60.8) (end 73.434994 59.6) (width 0.25) (layer "B.Cu") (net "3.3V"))
 (segment (start 72.350499 61.775499) (end 74.524501 61.775499) (width 0.25) (layer "B.Cu") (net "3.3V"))
 (segment (start 73.2 59.7) (end 73.3 59.6) (width 0.25) (layer "B.Cu") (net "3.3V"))
 (segment (start 73.434994 59.6) (end 73.3 59.6) (width 0.25) (layer "B.Cu") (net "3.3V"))
 (segment (start 78 64.1) (end 74.8 67.3) (width 0.25) (layer "B.Cu") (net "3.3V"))
 (segment (start 66.9 59) (end 66.9 58.6) (width 0.25) (layer "B.Cu") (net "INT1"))
 (segment (start 64.6 67.8) (end 66.3 66.1) (width 0.25) (layer "B.Cu") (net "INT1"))
 (segment (start 66.9 59.6) (end 66.9 59) (width 0.25) (layer "B.Cu") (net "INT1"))
 (segment (start 66.9 58.6) (end 67.9 57.6) (width 0.25) (layer "B.Cu") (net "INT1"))
 (segment (start 66.3 66.1) (end 66.3 60.2) (width 0.25) (layer "B.Cu") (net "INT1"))
 (segment (start 66.3 60.2) (end 66.9 59.6) (width 0.25) (layer "B.Cu") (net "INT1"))
 (segment (start 67.8 60.5) (end 68.6 59.7) (width 0.25) (layer "B.Cu") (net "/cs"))
 (segment (start 67.1 60.5) (end 67.8 60.5) (width 0.25) (layer "B.Cu") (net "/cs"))
 (segment (start 67.72452 62.67548) (end 67.72452 61.12452) (width 0.25) (layer "B.Cu") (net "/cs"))
 (segment (start 67.72452 61.12452) (end 67.1 60.5) (width 0.25) (layer "B.Cu") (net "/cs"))
 (segment (start 68.6 59.7) (end 69.775 59.7) (width 0.25) (layer "B.Cu") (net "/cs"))
 (segment (start 67.1 63.3) (end 67.72452 62.67548) (width 0.25) (layer "B.Cu") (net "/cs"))
 (segment (start 79.1125 63.9875) (end 79 64.1) (width 0.25) (layer "B.Cu") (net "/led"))
 (segment (start 81 63.9875) (end 79.1125 63.9875) (width 0.25) (layer "B.Cu") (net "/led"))
 (segment (start 70.7 58.1) (end 71 58.4) (width 0.25) (layer "B.Cu") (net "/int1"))
 (segment (start 71 58.4) (end 71 58.975) (width 0.25) (layer "B.Cu") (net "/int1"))
 (segment (start 69.3 58.1) (end 70.7 58.1) (width 0.25) (layer "B.Cu") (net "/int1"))
 (segment (start 67.9 59) (end 68.4 59) (width 0.25) (layer "B.Cu") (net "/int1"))
 (segment (start 68.4 59) (end 69.3 58.1) (width 0.25) (layer "B.Cu") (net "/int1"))
 (segment (start 69.775 60.2) (end 68.9 60.2) (width 0.25) (layer "B.Cu") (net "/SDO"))
 (segment (start 68.9 60.2) (end 68.3 60.8) (width 0.25) (layer "B.Cu") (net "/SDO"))
 (segment (start 68.3 60.8) (end 68.3 63.3) (width 0.25) (layer "B.Cu") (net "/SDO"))
 (segment (start 68.9 62.7) (end 69.5 63.3) (width 0.25) (layer "B.Cu") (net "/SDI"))
 (segment (start 69.2 60.7) (end 68.9 61) (width 0.25) (layer "B.Cu") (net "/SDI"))
 (segment (start 69.775 60.7) (end 69.2 60.7) (width 0.25) (layer "B.Cu") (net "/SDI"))
 (segment (start 68.9 61) (end 68.9 62.7) (width 0.25) (layer "B.Cu") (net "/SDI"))
 (segment (start 70.5 61.425) (end 70.5 62) (width 0.25) (layer "B.Cu") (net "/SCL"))
 (segment (start 70.5 62) (end 71.5 63) (width 0.25) (layer "B.Cu") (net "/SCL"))
 (segment (start 71.5 63) (end 71.5 63.3) (width 0.25) (layer "B.Cu") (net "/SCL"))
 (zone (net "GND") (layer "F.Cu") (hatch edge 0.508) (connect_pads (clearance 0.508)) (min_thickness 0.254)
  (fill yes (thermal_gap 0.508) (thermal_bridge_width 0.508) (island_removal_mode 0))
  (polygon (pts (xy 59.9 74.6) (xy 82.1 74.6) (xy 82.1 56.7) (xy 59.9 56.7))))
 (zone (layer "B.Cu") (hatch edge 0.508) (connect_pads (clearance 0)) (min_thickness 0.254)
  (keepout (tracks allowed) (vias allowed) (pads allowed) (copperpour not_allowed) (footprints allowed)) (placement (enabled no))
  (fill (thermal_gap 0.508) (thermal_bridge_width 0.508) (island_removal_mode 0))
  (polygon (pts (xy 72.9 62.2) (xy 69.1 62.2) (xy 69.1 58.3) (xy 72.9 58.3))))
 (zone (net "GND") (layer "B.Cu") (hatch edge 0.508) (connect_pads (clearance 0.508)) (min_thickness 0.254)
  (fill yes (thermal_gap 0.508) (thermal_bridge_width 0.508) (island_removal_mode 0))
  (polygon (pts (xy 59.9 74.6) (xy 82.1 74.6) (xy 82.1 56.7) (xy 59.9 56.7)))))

